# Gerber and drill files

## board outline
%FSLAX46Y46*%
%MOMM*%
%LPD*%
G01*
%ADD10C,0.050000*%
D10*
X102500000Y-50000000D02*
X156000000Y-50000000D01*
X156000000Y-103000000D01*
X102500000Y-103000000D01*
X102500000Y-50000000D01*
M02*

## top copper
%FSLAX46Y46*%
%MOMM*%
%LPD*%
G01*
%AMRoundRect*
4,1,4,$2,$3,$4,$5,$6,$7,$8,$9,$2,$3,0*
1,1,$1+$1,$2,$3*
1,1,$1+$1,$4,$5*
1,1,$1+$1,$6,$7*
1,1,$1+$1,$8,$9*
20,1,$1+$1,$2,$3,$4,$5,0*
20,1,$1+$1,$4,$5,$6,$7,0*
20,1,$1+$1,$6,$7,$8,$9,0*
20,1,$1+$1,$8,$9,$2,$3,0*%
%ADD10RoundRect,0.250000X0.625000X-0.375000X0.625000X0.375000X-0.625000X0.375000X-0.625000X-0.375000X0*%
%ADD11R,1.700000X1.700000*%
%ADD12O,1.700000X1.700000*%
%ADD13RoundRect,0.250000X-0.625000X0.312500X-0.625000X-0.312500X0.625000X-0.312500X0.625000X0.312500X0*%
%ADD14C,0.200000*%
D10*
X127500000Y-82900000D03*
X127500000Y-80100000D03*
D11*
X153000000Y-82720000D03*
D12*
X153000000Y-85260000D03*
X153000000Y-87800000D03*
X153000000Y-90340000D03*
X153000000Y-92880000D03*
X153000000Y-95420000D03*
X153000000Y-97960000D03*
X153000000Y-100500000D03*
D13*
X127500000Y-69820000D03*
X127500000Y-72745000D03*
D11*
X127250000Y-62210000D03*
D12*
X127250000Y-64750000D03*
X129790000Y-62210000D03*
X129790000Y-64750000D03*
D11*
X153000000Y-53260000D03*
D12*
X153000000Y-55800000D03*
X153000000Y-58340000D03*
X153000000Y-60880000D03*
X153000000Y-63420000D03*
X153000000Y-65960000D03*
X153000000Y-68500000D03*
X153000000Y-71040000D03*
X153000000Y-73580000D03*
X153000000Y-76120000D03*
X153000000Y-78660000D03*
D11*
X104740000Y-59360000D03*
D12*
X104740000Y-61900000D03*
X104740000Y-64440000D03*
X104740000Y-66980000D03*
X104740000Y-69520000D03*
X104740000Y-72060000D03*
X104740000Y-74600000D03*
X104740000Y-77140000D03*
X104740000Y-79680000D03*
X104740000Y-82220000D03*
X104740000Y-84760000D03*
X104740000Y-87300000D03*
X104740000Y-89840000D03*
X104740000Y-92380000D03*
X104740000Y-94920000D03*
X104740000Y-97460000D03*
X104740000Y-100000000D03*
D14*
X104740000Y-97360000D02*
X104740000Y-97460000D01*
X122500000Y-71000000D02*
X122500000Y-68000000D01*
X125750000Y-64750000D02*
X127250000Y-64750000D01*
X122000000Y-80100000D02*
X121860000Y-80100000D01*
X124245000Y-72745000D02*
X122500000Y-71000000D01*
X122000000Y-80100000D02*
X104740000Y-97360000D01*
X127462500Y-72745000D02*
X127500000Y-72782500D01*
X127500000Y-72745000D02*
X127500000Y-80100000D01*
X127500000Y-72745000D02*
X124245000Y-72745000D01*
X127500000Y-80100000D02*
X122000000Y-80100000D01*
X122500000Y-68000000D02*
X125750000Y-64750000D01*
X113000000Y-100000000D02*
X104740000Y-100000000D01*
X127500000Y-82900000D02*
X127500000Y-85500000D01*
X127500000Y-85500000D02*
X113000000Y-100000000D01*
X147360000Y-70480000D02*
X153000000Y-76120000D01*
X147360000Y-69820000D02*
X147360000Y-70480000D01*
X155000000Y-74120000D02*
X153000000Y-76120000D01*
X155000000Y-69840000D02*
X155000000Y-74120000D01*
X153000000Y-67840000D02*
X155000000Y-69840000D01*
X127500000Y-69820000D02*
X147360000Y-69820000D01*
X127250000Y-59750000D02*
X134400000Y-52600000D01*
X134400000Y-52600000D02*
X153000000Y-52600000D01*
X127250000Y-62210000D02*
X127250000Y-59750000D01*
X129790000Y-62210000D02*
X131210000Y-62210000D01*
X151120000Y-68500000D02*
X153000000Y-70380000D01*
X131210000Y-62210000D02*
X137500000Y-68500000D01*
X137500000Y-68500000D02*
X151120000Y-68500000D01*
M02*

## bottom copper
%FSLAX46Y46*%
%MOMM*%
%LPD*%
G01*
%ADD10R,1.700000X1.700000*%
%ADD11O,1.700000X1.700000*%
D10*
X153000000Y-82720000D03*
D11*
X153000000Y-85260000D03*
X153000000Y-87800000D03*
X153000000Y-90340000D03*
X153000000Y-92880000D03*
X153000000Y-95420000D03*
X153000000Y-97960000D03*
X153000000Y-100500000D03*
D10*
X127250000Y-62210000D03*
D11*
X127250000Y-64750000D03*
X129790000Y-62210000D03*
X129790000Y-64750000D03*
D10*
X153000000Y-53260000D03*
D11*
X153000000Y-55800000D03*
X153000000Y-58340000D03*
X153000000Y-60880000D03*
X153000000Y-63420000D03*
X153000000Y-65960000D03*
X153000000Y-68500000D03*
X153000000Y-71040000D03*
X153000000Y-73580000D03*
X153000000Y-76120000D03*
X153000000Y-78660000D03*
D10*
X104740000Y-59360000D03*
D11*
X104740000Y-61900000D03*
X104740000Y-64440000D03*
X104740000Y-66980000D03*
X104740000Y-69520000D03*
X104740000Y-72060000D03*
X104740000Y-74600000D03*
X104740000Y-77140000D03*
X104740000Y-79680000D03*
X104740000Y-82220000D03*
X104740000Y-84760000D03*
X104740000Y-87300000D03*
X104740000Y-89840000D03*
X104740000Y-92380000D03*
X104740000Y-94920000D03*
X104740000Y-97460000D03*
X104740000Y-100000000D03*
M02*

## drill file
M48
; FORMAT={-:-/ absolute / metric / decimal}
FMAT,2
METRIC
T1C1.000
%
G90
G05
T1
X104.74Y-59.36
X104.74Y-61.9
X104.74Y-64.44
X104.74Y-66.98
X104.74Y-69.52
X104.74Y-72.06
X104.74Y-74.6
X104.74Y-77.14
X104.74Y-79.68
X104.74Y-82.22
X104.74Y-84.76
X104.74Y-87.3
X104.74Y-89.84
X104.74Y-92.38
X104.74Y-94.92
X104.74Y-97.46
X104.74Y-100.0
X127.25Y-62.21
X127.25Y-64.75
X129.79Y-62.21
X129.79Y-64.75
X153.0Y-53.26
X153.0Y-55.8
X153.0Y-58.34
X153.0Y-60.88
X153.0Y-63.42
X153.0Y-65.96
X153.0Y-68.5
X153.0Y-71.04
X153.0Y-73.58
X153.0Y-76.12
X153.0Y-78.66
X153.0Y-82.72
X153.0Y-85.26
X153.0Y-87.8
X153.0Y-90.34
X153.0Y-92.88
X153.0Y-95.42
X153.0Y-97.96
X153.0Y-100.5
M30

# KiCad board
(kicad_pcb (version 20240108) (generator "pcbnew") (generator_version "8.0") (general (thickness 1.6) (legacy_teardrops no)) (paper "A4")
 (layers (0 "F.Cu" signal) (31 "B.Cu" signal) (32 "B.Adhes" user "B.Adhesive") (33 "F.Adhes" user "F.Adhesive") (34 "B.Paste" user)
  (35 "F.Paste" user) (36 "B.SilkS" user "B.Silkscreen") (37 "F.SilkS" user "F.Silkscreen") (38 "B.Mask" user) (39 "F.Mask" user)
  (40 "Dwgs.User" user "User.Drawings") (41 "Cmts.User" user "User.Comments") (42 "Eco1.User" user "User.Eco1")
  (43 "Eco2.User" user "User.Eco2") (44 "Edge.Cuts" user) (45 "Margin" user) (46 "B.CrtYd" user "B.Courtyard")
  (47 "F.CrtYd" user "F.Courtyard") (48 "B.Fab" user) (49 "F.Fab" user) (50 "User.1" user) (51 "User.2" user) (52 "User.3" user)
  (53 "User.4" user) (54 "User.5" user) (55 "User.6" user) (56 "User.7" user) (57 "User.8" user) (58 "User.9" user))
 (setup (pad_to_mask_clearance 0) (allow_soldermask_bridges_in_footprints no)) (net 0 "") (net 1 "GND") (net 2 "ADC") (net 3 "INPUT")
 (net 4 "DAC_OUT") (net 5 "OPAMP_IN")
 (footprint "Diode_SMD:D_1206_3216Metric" (layer "F.Cu") (at 127.5 81.5 90)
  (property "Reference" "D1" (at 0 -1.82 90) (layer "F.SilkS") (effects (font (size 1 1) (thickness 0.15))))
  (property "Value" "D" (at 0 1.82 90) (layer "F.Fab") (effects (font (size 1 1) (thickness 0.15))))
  (pad "1" smd roundrect (at -1.4 0 90) (size 1.25 1.75) (layers "F.Cu" "F.Paste" "F.Mask") (roundrect_rratio 0.2) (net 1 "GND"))
  (pad "2" smd roundrect (at 1.4 0 90) (size 1.25 1.75) (layers "F.Cu" "F.Paste" "F.Mask") (roundrect_rratio 0.2) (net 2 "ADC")))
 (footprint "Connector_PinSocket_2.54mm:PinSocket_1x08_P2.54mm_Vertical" (layer "F.Cu") (at 153 82.72)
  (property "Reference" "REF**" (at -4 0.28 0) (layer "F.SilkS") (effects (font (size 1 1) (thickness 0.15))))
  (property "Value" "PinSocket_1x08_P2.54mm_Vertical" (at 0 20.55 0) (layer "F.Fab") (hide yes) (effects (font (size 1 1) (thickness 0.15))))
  (pad "1" thru_hole rect (at 0 0) (size 1.7 1.7) (drill 1) (layers "*.Cu" "*.Mask") (remove_unused_layers no))
  (pad "2" thru_hole oval (at 0 2.54) (size 1.7 1.7) (drill 1) (layers "*.Cu" "*.Mask") (remove_unused_layers no))
  (pad "3" thru_hole oval (at 0 5.08) (size 1.7 1.7) (drill 1) (layers "*.Cu" "*.Mask") (remove_unused_layers no))
  (pad "4" thru_hole oval (at 0 7.62) (size 1.7 1.7) (drill 1) (layers "*.Cu" "*.Mask") (remove_unused_layers no))
  (pad "5" thru_hole oval (at 0 10.16) (size 1.7 1.7) (drill 1) (layers "*.Cu" "*.Mask") (remove_unused_layers no))
  (pad "6" thru_hole oval (at 0 12.7) (size 1.7 1.7) (drill 1) (layers "*.Cu" "*.Mask") (remove_unused_layers no))
  (pad "7" thru_hole oval (at 0 15.24) (size 1.7 1.7) (drill 1) (layers "*.Cu" "*.Mask") (remove_unused_layers no))
  (pad "8" thru_hole oval (at 0 17.78) (size 1.7 1.7) (drill 1) (layers "*.Cu" "*.Mask") (remove_unused_layers no)))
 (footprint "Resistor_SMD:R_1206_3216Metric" (layer "F.Cu") (at 127.5 71.2825 -90)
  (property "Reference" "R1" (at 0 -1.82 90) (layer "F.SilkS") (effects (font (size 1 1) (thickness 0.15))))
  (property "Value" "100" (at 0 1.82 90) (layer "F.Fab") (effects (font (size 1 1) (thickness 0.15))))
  (pad "1" smd roundrect (at -1.4625 0 270) (size 1.125 1.75) (layers "F.Cu" "F.Paste" "F.Mask") (roundrect_rratio 0.222222) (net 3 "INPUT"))
  (pad "2" smd roundrect (at 1.4625 0 270) (size 1.125 1.75) (layers "F.Cu" "F.Paste" "F.Mask") (roundrect_rratio 0.222222) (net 2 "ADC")))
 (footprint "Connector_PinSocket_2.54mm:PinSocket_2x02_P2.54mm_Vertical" (layer "F.Cu") (at 127.25 62.21 90)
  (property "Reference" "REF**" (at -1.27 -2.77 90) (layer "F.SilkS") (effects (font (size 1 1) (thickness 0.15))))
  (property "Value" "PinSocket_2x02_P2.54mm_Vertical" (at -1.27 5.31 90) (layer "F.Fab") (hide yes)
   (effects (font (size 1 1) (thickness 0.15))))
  (pad "1" thru_hole rect (at 0 0 90) (size 1.7 1.7) (drill 1) (layers "*.Cu" "*.Mask") (remove_unused_layers no) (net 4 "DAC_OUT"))
  (pad "2" thru_hole oval (at -2.54 0 90) (size 1.7 1.7) (drill 1) (layers "*.Cu" "*.Mask") (remove_unused_layers no) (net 2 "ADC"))
  (pad "3" thru_hole oval (at 0 2.54 90) (size 1.7 1.7) (drill 1) (layers "*.Cu" "*.Mask") (remove_unused_layers no) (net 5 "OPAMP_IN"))
  (pad "4" thru_hole oval (at -2.54 2.54 90) (size 1.7 1.7) (drill 1) (layers "*.Cu" "*.Mask") (remove_unused_layers no)))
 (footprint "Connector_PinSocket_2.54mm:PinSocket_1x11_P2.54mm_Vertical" (layer "F.Cu") (at 153 53.26)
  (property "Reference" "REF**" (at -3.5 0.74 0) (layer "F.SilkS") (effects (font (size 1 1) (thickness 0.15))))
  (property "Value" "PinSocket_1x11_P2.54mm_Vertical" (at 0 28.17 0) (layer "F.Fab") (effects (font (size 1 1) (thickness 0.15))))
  (pad "1" thru_hole rect (at 0 0) (size 1.7 1.7) (drill 1) (layers "*.Cu" "*.Mask") (remove_unused_layers no) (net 4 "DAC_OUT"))
  (pad "2" thru_hole oval (at 0 2.54) (size 1.7 1.7) (drill 1) (layers "*.Cu" "*.Mask") (remove_unused_layers no))
  (pad "3" thru_hole oval (at 0 5.08) (size 1.7 1.7) (drill 1) (layers "*.Cu" "*.Mask") (remove_unused_layers no))
  (pad "4" thru_hole oval (at 0 7.62) (size 1.7 1.7) (drill 1) (layers "*.Cu" "*.Mask") (remove_unused_layers no))
  (pad "5" thru_hole oval (at 0 10.16) (size 1.7 1.7) (drill 1) (layers "*.Cu" "*.Mask") (remove_unused_layers no))
  (pad "6" thru_hole oval (at 0 12.7) (size 1.7 1.7) (drill 1) (layers "*.Cu" "*.Mask") (remove_unused_layers no))
  (pad "7" thru_hole oval (at 0 15.24) (size 1.7 1.7) (drill 1) (layers "*.Cu" "*.Mask") (remove_unused_layers no) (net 3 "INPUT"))
  (pad "8" thru_hole oval (at 0 17.78) (size 1.7 1.7) (drill 1) (layers "*.Cu" "*.Mask") (remove_unused_layers no) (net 5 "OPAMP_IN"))
  (pad "9" thru_hole oval (at 0 20.32) (size 1.7 1.7) (drill 1) (layers "*.Cu" "*.Mask") (remove_unused_layers no))
  (pad "10" thru_hole oval (at 0 22.86) (size 1.7 1.7) (drill 1) (layers "*.Cu" "*.Mask") (remove_unused_layers no) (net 3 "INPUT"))
  (pad "11" thru_hole oval (at 0 25.4) (size 1.7 1.7) (drill 1) (layers "*.Cu" "*.Mask") (remove_unused_layers no)))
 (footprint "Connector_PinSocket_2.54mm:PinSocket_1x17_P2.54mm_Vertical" (layer "F.Cu") (at 104.74 59.36)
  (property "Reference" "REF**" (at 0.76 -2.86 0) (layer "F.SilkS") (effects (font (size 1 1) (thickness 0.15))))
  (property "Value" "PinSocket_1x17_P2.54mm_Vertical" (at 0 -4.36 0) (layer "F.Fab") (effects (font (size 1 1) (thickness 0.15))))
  (pad "1" thru_hole rect (at 0 0) (size 1.7 1.7) (drill 1) (layers "*.Cu" "*.Mask") (remove_unused_layers no))
  (pad "2" thru_hole oval (at 0 2.54) (size 1.7 1.7) (drill 1) (layers "*.Cu" "*.Mask") (remove_unused_layers no))
  (pad "3" thru_hole oval (at 0 5.08) (size 1.7 1.7) (drill 1) (layers "*.Cu" "*.Mask") (remove_unused_layers no))
  (pad "4" thru_hole oval (at 0 7.62) (size 1.7 1.7) (drill 1) (layers "*.Cu" "*.Mask") (remove_unused_layers no))
  (pad "5" thru_hole oval (at 0 10.16) (size 1.7 1.7) (drill 1) (layers "*.Cu" "*.Mask") (remove_unused_layers no))
  (pad "6" thru_hole oval (at 0 12.7) (size 1.7 1.7) (drill 1) (layers "*.Cu" "*.Mask") (remove_unused_layers no))
  (pad "7" thru_hole oval (at 0 15.24) (size 1.7 1.7) (drill 1) (layers "*.Cu" "*.Mask") (remove_unused_layers no))
  (pad "8" thru_hole oval (at 0 17.78) (size 1.7 1.7) (drill 1) (layers "*.Cu" "*.Mask") (remove_unused_layers no))
  (pad "9" thru_hole oval (at 0 20.32) (size 1.7 1.7) (drill 1) (layers "*.Cu" "*.Mask") (remove_unused_layers no))
  (pad "10" thru_hole oval (at 0 22.86) (size 1.7 1.7) (drill 1) (layers "*.Cu" "*.Mask") (remove_unused_layers no))
  (pad "11" thru_hole oval (at 0 25.4) (size 1.7 1.7) (drill 1) (layers "*.Cu" "*.Mask") (remove_unused_layers no))
  (pad "12" thru_hole oval (at 0 27.94) (size 1.7 1.7) (drill 1) (layers "*.Cu" "*.Mask") (remove_unused_layers no))
  (pad "13" thru_hole oval (at 0 30.48) (size 1.7 1.7) (drill 1) (layers "*.Cu" "*.Mask") (remove_unused_layers no))
  (pad "14" thru_hole oval (at 0 33.02) (size 1.7 1.7) (drill 1) (layers "*.Cu" "*.Mask") (remove_unused_layers no))
  (pad "15" thru_hole oval (at 0 35.56) (size 1.7 1.7) (drill 1) (layers "*.Cu" "*.Mask") (remove_unused_layers no))
  (pad "16" thru_hole oval (at 0 38.1) (size 1.7 1.7) (drill 1) (layers "*.Cu" "*.Mask") (remove_unused_layers no) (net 2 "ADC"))
  (pad "17" thru_hole oval (at 0 40.64) (size 1.7 1.7) (drill 1) (layers "*.Cu" "*.Mask") (remove_unused_layers no) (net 1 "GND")))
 (gr_rect (start 102.5 50) (end 156 103) (stroke (width 0.05) (type default)) (fill none) (layer "Edge.Cuts"))
 (segment (start 104.74 97.36) (end 104.74 97.46) (width 0.2) (layer "F.Cu") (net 2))
 (segment (start 122.5 71) (end 122.5 68) (width 0.2) (layer "F.Cu") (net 2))
 (segment (start 125.75 64.75) (end 127.25 64.75) (width 0.2) (layer "F.Cu") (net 2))
 (segment (start 122 80.1) (end 121.86 80.1) (width 0.2) (layer "F.Cu") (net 2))
 (segment (start 124.245 72.745) (end 122.5 71) (width 0.2) (layer "F.Cu") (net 2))
 (segment (start 122 80.1) (end 104.74 97.36) (width 0.2) (layer "F.Cu") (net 2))
 (segment (start 127.4625 72.745) (end 127.5 72.7825) (width 0.2) (layer "F.Cu") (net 2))
 (segment (start 127.5 72.745) (end 127.5 80.1) (width 0.2) (layer "F.Cu") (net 2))
 (segment (start 127.5 72.745) (end 124.245 72.745) (width 0.2) (layer "F.Cu") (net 2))
 (segment (start 127.5 80.1) (end 122 80.1) (width 0.2) (layer "F.Cu") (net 2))
 (segment (start 122.5 68) (end 125.75 64.75) (width 0.2) (layer "F.Cu") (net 2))
 (segment (start 113 100) (end 104.74 100) (width 0.2) (layer "F.Cu") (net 1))
 (segment (start 127.5 82.9) (end 127.5 85.5) (width 0.2) (layer "F.Cu") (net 1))
 (segment (start 127.5 85.5) (end 113 100) (width 0.2) (layer "F.Cu") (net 1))
 (segment (start 147.36 70.48) (end 153 76.12) (width 0.2) (layer "F.Cu") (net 3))
 (segment (start 147.36 69.82) (end 147.36 70.48) (width 0.2) (layer "F.Cu") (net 3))
 (segment (start 155 74.12) (end 153 76.12) (width 0.2) (layer "F.Cu") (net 3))
 (segment (start 155 69.84) (end 155 74.12) (width 0.2) (layer "F.Cu") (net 3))
 (segment (start 153 67.84) (end 155 69.84) (width 0.2) (layer "F.Cu") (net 3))
 (segment (start 127.5 69.82) (end 147.36 69.82) (width 0.2) (layer "F.Cu") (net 3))
 (segment (start 127.25 59.75) (end 134.4 52.6) (width 0.2) (layer "F.Cu") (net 4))
 (segment (start 134.4 52.6) (end 153 52.6) (width 0.2) (layer "F.Cu") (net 4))
 (segment (start 127.25 62.21) (end 127.25 59.75) (width 0.2) (layer "F.Cu") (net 4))
 (segment (start 129.79 62.21) (end 131.21 62.21) (width 0.2) (layer "F.Cu") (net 5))
 (segment (start 151.12 68.5) (end 153 70.38) (width 0.2) (layer "F.Cu") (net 5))
 (segment (start 131.21 62.21) (end 137.5 68.5) (width 0.2) (layer "F.Cu") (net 5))
 (segment (start 137.5 68.5) (end 151.12 68.5) (width 0.2) (layer "F.Cu") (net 5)))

